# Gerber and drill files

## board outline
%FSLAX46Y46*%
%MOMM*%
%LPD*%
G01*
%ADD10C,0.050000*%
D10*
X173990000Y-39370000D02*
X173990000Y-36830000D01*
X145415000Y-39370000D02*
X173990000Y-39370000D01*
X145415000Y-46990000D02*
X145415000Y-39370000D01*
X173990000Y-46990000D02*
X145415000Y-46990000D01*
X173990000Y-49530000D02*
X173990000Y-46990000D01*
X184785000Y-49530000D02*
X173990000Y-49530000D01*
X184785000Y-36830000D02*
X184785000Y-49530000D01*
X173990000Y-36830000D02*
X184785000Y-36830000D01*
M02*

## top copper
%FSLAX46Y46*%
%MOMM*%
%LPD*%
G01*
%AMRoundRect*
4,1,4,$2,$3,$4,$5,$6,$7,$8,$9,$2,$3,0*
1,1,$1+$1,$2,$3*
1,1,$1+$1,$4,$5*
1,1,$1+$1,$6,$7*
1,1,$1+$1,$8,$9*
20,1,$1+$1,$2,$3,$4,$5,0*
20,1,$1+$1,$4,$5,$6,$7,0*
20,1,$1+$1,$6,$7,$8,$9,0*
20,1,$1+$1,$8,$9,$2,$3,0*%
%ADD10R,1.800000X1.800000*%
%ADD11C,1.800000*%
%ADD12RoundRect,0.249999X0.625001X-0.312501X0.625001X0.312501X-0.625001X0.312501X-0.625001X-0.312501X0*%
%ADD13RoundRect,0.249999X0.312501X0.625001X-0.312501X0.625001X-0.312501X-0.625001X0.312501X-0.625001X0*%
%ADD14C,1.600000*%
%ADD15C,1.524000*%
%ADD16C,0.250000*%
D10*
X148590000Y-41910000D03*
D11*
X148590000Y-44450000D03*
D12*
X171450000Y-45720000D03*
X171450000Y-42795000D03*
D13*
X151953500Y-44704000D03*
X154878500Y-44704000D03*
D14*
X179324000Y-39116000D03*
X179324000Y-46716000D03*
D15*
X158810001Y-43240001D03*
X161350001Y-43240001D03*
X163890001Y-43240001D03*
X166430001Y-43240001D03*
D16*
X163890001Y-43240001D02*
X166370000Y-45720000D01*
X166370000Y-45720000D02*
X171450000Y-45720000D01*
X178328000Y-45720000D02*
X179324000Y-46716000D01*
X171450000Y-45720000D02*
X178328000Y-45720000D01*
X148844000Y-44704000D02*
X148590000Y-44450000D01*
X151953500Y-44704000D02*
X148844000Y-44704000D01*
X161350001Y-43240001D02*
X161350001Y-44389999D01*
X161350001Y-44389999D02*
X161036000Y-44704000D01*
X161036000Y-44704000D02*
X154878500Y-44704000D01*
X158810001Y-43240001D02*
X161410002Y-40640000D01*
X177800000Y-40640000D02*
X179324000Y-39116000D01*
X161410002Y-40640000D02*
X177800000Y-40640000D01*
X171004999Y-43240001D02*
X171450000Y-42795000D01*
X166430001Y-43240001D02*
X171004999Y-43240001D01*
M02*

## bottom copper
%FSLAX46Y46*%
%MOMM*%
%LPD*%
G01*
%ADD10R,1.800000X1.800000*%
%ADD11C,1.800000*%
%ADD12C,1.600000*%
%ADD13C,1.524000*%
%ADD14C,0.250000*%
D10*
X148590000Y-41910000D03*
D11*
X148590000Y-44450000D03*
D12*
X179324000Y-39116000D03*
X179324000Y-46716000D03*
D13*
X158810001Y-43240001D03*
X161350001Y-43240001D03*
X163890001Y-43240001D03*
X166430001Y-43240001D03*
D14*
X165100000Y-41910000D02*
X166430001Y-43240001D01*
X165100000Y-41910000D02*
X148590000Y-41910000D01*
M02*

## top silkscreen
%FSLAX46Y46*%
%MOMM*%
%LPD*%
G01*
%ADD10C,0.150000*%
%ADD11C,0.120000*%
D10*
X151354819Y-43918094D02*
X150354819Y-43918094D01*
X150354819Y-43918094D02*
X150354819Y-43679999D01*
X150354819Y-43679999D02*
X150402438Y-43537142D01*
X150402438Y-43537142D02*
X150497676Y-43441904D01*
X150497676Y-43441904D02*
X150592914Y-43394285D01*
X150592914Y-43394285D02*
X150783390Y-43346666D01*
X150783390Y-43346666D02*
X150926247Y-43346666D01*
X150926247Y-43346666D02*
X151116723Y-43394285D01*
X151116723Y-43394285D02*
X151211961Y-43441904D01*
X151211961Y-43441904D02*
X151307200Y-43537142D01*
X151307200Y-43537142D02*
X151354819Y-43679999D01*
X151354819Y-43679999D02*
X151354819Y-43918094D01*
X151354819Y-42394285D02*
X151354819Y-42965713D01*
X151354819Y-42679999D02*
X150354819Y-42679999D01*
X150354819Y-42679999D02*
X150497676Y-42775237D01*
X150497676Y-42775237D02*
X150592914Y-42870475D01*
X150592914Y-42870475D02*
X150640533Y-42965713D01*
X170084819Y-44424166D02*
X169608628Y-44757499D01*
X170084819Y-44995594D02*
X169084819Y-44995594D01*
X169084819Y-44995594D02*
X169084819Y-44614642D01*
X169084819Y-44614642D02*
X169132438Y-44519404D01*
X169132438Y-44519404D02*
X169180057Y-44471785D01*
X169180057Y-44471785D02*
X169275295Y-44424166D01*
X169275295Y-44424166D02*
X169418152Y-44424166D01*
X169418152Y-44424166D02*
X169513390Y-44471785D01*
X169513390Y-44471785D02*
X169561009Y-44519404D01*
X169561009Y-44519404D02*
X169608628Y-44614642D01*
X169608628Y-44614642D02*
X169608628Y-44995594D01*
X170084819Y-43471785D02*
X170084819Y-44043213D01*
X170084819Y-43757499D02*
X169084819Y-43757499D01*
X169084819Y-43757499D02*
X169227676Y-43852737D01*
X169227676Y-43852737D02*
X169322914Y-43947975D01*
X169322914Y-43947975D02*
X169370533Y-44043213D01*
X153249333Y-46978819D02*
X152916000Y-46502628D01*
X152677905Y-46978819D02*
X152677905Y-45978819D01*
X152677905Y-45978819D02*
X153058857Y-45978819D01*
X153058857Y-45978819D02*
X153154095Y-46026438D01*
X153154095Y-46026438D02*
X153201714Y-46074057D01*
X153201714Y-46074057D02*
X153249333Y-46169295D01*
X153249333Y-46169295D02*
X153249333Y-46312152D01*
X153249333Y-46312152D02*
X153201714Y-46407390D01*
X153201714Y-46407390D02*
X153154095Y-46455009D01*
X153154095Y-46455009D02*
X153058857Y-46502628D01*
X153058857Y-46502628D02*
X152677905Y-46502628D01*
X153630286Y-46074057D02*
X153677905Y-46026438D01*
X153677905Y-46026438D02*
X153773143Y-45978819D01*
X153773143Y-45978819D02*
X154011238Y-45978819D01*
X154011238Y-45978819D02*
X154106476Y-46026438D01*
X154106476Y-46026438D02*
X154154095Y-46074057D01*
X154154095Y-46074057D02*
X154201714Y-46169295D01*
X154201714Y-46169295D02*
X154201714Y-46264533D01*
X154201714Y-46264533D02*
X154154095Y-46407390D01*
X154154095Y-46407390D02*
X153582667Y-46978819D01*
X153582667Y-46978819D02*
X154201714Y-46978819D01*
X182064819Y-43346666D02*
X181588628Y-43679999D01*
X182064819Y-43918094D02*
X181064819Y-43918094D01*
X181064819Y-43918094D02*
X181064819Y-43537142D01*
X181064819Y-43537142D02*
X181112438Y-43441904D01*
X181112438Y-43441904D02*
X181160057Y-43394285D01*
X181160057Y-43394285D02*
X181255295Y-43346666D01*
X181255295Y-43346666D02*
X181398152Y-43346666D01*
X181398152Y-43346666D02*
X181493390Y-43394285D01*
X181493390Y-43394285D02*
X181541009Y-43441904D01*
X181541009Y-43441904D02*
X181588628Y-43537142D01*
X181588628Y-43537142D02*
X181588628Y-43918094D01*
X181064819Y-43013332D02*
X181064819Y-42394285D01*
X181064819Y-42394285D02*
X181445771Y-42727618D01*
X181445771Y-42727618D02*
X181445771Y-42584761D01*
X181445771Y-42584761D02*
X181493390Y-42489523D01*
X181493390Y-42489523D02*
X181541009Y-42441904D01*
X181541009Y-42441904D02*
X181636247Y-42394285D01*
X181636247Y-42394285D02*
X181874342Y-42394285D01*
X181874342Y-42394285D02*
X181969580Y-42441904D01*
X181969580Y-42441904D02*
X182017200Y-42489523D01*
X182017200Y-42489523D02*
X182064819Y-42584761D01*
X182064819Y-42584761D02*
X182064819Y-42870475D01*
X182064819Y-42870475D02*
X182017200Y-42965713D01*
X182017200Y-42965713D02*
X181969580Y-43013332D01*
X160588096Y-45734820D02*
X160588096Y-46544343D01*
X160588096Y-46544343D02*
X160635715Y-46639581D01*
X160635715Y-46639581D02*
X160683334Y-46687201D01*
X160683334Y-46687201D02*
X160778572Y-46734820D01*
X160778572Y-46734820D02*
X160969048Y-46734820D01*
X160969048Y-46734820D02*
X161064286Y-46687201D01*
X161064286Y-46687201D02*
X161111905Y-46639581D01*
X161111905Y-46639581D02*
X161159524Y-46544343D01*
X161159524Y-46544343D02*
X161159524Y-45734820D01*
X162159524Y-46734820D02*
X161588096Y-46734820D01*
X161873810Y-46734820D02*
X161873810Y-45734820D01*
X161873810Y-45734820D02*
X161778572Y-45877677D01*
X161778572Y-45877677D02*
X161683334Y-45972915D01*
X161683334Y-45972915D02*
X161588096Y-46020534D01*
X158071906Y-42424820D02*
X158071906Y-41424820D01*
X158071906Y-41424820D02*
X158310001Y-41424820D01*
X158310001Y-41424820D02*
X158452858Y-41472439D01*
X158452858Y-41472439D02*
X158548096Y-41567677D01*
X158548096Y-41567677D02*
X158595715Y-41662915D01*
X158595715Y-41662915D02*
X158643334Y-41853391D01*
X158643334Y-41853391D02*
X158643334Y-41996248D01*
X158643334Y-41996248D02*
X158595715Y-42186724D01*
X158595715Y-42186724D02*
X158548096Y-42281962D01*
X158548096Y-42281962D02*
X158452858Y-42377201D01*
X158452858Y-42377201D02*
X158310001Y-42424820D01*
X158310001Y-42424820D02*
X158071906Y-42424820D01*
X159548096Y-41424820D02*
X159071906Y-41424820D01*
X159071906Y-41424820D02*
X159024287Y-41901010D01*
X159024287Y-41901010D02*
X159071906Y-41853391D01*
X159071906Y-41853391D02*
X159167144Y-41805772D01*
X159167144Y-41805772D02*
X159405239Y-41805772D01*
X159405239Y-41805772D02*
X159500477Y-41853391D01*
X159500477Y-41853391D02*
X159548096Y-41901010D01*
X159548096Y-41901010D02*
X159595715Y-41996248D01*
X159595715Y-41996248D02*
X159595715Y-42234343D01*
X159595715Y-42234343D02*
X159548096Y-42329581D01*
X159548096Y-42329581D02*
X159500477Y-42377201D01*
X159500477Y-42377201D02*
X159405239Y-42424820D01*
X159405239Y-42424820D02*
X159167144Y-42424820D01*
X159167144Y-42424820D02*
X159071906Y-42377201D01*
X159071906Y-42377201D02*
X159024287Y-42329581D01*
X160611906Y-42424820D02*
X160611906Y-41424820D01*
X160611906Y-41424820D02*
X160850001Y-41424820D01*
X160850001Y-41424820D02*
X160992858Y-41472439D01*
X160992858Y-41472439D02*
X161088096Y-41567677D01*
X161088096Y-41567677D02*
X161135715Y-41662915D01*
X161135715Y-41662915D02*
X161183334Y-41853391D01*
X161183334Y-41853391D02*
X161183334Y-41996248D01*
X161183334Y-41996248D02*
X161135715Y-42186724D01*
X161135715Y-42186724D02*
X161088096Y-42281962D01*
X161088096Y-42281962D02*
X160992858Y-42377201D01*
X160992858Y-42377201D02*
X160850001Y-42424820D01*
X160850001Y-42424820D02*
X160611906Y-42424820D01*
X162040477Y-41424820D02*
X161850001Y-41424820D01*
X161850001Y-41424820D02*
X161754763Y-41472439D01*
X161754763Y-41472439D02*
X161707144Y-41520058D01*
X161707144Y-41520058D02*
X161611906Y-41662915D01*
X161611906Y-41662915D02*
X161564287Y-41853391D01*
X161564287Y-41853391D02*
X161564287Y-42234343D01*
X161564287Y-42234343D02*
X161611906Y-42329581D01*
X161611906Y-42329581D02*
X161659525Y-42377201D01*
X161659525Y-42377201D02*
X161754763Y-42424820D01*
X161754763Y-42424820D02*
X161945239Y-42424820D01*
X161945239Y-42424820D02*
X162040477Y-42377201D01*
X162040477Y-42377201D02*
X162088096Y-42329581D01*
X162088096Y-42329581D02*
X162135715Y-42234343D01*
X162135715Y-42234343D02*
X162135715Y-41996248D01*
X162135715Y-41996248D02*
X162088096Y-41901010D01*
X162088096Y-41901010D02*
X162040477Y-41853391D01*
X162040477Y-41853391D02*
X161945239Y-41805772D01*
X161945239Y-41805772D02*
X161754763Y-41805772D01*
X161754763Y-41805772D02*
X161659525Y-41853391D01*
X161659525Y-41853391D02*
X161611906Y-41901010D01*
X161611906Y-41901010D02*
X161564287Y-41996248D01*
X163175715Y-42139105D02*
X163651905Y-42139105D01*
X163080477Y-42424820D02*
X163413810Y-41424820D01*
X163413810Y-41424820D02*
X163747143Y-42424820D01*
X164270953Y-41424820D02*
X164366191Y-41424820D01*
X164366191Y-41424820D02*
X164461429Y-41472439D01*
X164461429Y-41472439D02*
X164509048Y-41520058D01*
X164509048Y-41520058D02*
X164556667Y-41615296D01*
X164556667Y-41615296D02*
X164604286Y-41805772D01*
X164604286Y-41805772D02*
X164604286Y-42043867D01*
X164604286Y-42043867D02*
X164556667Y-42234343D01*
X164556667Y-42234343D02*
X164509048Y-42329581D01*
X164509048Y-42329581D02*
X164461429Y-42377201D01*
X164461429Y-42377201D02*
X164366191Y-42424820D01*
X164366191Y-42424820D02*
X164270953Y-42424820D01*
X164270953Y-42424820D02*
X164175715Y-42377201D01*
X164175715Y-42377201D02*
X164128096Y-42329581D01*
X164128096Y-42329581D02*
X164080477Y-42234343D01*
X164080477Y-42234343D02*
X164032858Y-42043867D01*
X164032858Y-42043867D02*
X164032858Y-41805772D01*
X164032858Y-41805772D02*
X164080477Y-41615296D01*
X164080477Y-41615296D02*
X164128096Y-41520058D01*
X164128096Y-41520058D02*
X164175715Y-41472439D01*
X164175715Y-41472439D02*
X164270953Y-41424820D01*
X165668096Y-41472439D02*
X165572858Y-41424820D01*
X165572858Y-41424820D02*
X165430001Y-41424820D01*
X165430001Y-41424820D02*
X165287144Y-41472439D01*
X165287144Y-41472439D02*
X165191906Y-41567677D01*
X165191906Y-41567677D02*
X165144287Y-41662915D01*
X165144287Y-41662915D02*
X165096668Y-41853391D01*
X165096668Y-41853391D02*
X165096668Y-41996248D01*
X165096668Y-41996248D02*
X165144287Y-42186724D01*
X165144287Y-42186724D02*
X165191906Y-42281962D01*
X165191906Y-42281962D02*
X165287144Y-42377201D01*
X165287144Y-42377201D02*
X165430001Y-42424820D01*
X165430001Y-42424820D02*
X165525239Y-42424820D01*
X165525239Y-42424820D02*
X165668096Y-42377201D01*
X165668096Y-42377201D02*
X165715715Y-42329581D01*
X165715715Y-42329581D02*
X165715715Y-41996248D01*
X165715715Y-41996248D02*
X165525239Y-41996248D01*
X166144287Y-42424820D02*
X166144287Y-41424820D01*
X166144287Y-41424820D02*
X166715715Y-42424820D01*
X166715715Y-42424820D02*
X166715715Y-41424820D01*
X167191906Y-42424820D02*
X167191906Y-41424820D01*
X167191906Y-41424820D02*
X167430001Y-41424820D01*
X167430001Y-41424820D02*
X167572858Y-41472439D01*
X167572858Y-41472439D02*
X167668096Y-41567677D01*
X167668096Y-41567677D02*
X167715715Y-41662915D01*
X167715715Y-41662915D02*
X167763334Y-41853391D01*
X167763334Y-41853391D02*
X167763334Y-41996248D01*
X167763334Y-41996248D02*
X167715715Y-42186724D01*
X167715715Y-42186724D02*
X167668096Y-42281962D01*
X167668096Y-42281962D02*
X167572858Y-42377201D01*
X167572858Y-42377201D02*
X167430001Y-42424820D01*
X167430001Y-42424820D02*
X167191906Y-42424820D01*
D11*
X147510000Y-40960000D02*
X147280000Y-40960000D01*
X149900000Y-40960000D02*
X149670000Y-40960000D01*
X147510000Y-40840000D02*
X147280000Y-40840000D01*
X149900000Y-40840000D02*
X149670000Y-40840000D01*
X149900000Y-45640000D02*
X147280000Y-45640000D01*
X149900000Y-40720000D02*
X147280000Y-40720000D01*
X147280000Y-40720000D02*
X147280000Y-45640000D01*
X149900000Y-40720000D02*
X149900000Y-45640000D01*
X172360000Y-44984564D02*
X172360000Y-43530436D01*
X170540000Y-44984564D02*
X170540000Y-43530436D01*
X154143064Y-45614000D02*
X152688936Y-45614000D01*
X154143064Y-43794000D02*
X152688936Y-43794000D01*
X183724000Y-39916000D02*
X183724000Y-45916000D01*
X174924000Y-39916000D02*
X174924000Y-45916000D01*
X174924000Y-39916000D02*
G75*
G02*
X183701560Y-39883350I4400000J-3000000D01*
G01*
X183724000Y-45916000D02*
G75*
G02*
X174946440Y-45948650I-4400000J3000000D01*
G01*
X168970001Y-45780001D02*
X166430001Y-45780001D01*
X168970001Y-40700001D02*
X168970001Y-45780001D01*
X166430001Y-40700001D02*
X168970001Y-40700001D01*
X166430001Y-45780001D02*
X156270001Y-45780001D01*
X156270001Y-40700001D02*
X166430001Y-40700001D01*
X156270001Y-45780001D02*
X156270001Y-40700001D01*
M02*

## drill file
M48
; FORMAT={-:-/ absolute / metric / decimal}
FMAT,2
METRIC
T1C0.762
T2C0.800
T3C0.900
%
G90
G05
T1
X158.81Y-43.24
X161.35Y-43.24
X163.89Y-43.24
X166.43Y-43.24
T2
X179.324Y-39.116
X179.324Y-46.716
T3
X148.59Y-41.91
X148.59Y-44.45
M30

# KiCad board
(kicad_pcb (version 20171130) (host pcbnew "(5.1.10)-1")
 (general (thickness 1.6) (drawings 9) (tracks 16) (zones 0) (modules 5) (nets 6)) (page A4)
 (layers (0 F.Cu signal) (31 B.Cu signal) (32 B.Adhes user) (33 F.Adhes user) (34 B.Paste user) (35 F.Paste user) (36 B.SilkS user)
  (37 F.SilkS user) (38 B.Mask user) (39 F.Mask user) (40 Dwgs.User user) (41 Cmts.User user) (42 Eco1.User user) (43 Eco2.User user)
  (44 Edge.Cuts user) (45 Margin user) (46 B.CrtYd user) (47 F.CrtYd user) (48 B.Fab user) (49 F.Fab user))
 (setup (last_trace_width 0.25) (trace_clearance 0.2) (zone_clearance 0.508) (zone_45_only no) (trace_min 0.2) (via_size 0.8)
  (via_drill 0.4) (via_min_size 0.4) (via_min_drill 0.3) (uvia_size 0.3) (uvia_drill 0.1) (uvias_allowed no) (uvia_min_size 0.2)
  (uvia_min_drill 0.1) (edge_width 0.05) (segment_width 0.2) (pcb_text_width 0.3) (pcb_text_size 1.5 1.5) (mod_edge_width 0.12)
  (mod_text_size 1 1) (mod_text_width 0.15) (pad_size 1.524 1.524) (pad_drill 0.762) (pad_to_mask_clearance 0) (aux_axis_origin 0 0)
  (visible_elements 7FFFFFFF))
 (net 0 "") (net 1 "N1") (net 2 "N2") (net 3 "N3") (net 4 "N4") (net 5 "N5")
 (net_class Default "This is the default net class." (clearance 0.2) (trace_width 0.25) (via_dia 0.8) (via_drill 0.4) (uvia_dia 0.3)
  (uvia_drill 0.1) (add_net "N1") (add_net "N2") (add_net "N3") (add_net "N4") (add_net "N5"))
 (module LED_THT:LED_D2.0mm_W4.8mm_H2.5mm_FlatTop (layer F.Cu) (at 148.59 41.91 270)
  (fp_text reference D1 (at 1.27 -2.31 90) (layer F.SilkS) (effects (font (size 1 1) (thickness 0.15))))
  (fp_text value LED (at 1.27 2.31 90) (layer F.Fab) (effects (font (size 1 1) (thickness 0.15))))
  (fp_line (start -0.95 1.08) (end -0.95 1.31) (layer F.SilkS) (width 0.12))
  (fp_line (start -0.95 -1.31) (end -0.95 -1.08) (layer F.SilkS) (width 0.12))
  (fp_line (start -1.07 1.08) (end -1.07 1.31) (layer F.SilkS) (width 0.12))
  (fp_line (start -1.07 -1.31) (end -1.07 -1.08) (layer F.SilkS) (width 0.12))
  (fp_line (start 3.73 -1.31) (end 3.73 1.31) (layer F.SilkS) (width 0.12))
  (fp_line (start -1.19 -1.31) (end -1.19 1.31) (layer F.SilkS) (width 0.12))
  (fp_line (start -1.19 1.31) (end 3.73 1.31) (layer F.SilkS) (width 0.12))
  (fp_line (start -1.19 -1.31) (end 3.73 -1.31) (layer F.SilkS) (width 0.12))
  (pad 1 thru_hole rect (at 0 0 270) (size 1.8 1.8) (drill 0.9) (layers *.Cu *.Mask) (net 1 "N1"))
  (pad 2 thru_hole circle (at 2.54 0 270) (size 1.8 1.8) (drill 0.9) (layers *.Cu *.Mask) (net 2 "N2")))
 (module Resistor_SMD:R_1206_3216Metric (layer F.Cu) (at 171.45 44.2575 90)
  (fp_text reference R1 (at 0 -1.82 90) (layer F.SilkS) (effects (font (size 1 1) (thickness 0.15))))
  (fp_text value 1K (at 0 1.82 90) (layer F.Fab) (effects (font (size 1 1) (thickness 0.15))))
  (fp_line (start -0.727064 0.91) (end 0.727064 0.91) (layer F.SilkS) (width 0.12))
  (fp_line (start -0.727064 -0.91) (end 0.727064 -0.91) (layer F.SilkS) (width 0.12))
  (pad 1 smd roundrect (at -1.4625 0 90) (size 1.125 1.75) (layers F.Cu F.Paste F.Mask) (roundrect_rratio 0.2222213333333333) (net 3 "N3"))
  (pad 2 smd roundrect (at 1.4625 0 90) (size 1.125 1.75) (layers F.Cu F.Paste F.Mask) (roundrect_rratio 0.2222213333333333) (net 1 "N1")))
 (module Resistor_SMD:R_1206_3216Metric (layer F.Cu) (at 153.416 44.704 180)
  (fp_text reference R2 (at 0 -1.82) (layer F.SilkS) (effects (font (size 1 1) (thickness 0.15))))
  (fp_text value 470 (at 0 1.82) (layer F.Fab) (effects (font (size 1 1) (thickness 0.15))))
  (fp_line (start -0.727064 -0.91) (end 0.727064 -0.91) (layer F.SilkS) (width 0.12))
  (fp_line (start -0.727064 0.91) (end 0.727064 0.91) (layer F.SilkS) (width 0.12))
  (pad 2 smd roundrect (at 1.4625 0 180) (size 1.125 1.75) (layers F.Cu F.Paste F.Mask) (roundrect_rratio 0.2222213333333333) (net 2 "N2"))
  (pad 1 smd roundrect (at -1.4625 0 180) (size 1.125 1.75) (layers F.Cu F.Paste F.Mask) (roundrect_rratio 0.2222213333333333) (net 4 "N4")))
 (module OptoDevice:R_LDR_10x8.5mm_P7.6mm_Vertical (layer F.Cu) (at 179.324 39.116 270)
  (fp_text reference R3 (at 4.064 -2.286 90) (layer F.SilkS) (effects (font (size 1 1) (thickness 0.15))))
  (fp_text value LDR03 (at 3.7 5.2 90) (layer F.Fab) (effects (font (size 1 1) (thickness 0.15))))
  (fp_line (start 0.8 -4.4) (end 6.8 -4.4) (layer F.SilkS) (width 0.12))
  (fp_line (start 0.8 4.4) (end 6.8 4.4) (layer F.SilkS) (width 0.12))
  (fp_arc (start 3.8 0) (end 0.8 4.4) (angle 111) (layer F.SilkS) (width 0.12))
  (fp_arc (start 3.8 0) (end 6.8 -4.4) (angle 111) (layer F.SilkS) (width 0.12))
  (pad 1 thru_hole circle (at 0 0 270) (size 1.6 1.6) (drill 0.8) (layers *.Cu *.Mask) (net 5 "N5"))
  (pad 2 thru_hole circle (at 7.6 0 270) (size 1.6 1.6) (drill 0.8) (layers *.Cu *.Mask) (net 3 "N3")))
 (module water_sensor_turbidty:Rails (layer F.Cu) (at 161.350001 45.780001)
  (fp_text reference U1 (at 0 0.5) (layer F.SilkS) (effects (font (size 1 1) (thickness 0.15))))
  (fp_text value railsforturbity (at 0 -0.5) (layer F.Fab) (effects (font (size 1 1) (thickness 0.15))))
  (fp_line (start 7.62 0) (end 5.08 0) (layer F.SilkS) (width 0.12))
  (fp_line (start 7.62 -5.08) (end 7.62 0) (layer F.SilkS) (width 0.12))
  (fp_line (start 5.08 -5.08) (end 7.62 -5.08) (layer F.SilkS) (width 0.12))
  (fp_line (start 5.08 0) (end -5.08 0) (layer F.SilkS) (width 0.12))
  (fp_line (start -5.08 -5.08) (end 5.08 -5.08) (layer F.SilkS) (width 0.12))
  (fp_line (start -5.08 0) (end -5.08 -5.08) (layer F.SilkS) (width 0.12))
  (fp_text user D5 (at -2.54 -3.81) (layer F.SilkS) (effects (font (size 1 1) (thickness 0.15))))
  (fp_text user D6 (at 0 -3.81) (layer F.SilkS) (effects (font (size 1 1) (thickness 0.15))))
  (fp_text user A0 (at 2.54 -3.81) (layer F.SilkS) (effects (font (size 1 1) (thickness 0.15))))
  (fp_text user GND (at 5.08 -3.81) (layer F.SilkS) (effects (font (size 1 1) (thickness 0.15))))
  (pad 1 thru_hole circle (at -2.54 -2.54) (size 1.524 1.524) (drill 0.762) (layers *.Cu *.Mask) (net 5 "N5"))
  (pad 2 thru_hole circle (at 0 -2.54) (size 1.524 1.524) (drill 0.762) (layers *.Cu *.Mask) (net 4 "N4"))
  (pad 3 thru_hole circle (at 2.54 -2.54) (size 1.524 1.524) (drill 0.762) (layers *.Cu *.Mask) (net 3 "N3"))
  (pad 4 thru_hole circle (at 5.08 -2.54) (size 1.524 1.524) (drill 0.762) (layers *.Cu *.Mask) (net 1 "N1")))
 (gr_line (start 173.99 39.37) (end 173.99 36.83) (layer Edge.Cuts) (width 0.05))
 (gr_line (start 145.415 39.37) (end 173.99 39.37) (layer Edge.Cuts) (width 0.05))
 (gr_line (start 145.415 46.99) (end 145.415 39.37) (layer Edge.Cuts) (width 0.05))
 (gr_line (start 173.99 46.99) (end 145.415 46.99) (layer Edge.Cuts) (width 0.05))
 (gr_line (start 173.99 49.53) (end 173.99 46.99) (layer Edge.Cuts) (width 0.05))
 (gr_line (start 184.785 49.53) (end 173.99 49.53) (layer Edge.Cuts) (width 0.05))
 (gr_line (start 184.785 36.83) (end 184.785 49.53) (layer Edge.Cuts) (width 0.05))
 (gr_line (start 173.99 36.83) (end 184.785 36.83) (layer Edge.Cuts) (width 0.05))
 (segment (start 163.890001 43.240001) (end 166.37 45.72) (width 0.25) (layer F.Cu) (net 3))
 (segment (start 166.37 45.72) (end 171.45 45.72) (width 0.25) (layer F.Cu) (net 3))
 (segment (start 178.328 45.72) (end 179.324 46.716) (width 0.25) (layer F.Cu) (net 3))
 (segment (start 171.45 45.72) (end 178.328 45.72) (width 0.25) (layer F.Cu) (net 3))
 (segment (start 148.844 44.704) (end 148.59 44.45) (width 0.25) (layer F.Cu) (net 2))
 (segment (start 151.9535 44.704) (end 148.844 44.704) (width 0.25) (layer F.Cu) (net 2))
 (segment (start 161.350001 43.240001) (end 161.350001 44.389999) (width 0.25) (layer F.Cu) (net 4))
 (segment (start 161.350001 44.389999) (end 161.036 44.704) (width 0.25) (layer F.Cu) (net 4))
 (segment (start 161.036 44.704) (end 154.8785 44.704) (width 0.25) (layer F.Cu) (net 4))
 (segment (start 158.810001 43.240001) (end 161.410002 40.64) (width 0.25) (layer F.Cu) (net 5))
 (segment (start 177.8 40.64) (end 179.324 39.116) (width 0.25) (layer F.Cu) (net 5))
 (segment (start 161.410002 40.64) (end 177.8 40.64) (width 0.25) (layer F.Cu) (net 5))
 (segment (start 165.1 41.91) (end 166.430001 43.240001) (width 0.25) (layer B.Cu) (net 1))
 (segment (start 171.004999 43.240001) (end 171.45 42.795) (width 0.25) (layer F.Cu) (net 1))
 (segment (start 166.430001 43.240001) (end 171.004999 43.240001) (width 0.25) (layer F.Cu) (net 1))
 (segment (start 165.1 41.91) (end 148.59 41.91) (width 0.25) (layer B.Cu) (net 1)))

